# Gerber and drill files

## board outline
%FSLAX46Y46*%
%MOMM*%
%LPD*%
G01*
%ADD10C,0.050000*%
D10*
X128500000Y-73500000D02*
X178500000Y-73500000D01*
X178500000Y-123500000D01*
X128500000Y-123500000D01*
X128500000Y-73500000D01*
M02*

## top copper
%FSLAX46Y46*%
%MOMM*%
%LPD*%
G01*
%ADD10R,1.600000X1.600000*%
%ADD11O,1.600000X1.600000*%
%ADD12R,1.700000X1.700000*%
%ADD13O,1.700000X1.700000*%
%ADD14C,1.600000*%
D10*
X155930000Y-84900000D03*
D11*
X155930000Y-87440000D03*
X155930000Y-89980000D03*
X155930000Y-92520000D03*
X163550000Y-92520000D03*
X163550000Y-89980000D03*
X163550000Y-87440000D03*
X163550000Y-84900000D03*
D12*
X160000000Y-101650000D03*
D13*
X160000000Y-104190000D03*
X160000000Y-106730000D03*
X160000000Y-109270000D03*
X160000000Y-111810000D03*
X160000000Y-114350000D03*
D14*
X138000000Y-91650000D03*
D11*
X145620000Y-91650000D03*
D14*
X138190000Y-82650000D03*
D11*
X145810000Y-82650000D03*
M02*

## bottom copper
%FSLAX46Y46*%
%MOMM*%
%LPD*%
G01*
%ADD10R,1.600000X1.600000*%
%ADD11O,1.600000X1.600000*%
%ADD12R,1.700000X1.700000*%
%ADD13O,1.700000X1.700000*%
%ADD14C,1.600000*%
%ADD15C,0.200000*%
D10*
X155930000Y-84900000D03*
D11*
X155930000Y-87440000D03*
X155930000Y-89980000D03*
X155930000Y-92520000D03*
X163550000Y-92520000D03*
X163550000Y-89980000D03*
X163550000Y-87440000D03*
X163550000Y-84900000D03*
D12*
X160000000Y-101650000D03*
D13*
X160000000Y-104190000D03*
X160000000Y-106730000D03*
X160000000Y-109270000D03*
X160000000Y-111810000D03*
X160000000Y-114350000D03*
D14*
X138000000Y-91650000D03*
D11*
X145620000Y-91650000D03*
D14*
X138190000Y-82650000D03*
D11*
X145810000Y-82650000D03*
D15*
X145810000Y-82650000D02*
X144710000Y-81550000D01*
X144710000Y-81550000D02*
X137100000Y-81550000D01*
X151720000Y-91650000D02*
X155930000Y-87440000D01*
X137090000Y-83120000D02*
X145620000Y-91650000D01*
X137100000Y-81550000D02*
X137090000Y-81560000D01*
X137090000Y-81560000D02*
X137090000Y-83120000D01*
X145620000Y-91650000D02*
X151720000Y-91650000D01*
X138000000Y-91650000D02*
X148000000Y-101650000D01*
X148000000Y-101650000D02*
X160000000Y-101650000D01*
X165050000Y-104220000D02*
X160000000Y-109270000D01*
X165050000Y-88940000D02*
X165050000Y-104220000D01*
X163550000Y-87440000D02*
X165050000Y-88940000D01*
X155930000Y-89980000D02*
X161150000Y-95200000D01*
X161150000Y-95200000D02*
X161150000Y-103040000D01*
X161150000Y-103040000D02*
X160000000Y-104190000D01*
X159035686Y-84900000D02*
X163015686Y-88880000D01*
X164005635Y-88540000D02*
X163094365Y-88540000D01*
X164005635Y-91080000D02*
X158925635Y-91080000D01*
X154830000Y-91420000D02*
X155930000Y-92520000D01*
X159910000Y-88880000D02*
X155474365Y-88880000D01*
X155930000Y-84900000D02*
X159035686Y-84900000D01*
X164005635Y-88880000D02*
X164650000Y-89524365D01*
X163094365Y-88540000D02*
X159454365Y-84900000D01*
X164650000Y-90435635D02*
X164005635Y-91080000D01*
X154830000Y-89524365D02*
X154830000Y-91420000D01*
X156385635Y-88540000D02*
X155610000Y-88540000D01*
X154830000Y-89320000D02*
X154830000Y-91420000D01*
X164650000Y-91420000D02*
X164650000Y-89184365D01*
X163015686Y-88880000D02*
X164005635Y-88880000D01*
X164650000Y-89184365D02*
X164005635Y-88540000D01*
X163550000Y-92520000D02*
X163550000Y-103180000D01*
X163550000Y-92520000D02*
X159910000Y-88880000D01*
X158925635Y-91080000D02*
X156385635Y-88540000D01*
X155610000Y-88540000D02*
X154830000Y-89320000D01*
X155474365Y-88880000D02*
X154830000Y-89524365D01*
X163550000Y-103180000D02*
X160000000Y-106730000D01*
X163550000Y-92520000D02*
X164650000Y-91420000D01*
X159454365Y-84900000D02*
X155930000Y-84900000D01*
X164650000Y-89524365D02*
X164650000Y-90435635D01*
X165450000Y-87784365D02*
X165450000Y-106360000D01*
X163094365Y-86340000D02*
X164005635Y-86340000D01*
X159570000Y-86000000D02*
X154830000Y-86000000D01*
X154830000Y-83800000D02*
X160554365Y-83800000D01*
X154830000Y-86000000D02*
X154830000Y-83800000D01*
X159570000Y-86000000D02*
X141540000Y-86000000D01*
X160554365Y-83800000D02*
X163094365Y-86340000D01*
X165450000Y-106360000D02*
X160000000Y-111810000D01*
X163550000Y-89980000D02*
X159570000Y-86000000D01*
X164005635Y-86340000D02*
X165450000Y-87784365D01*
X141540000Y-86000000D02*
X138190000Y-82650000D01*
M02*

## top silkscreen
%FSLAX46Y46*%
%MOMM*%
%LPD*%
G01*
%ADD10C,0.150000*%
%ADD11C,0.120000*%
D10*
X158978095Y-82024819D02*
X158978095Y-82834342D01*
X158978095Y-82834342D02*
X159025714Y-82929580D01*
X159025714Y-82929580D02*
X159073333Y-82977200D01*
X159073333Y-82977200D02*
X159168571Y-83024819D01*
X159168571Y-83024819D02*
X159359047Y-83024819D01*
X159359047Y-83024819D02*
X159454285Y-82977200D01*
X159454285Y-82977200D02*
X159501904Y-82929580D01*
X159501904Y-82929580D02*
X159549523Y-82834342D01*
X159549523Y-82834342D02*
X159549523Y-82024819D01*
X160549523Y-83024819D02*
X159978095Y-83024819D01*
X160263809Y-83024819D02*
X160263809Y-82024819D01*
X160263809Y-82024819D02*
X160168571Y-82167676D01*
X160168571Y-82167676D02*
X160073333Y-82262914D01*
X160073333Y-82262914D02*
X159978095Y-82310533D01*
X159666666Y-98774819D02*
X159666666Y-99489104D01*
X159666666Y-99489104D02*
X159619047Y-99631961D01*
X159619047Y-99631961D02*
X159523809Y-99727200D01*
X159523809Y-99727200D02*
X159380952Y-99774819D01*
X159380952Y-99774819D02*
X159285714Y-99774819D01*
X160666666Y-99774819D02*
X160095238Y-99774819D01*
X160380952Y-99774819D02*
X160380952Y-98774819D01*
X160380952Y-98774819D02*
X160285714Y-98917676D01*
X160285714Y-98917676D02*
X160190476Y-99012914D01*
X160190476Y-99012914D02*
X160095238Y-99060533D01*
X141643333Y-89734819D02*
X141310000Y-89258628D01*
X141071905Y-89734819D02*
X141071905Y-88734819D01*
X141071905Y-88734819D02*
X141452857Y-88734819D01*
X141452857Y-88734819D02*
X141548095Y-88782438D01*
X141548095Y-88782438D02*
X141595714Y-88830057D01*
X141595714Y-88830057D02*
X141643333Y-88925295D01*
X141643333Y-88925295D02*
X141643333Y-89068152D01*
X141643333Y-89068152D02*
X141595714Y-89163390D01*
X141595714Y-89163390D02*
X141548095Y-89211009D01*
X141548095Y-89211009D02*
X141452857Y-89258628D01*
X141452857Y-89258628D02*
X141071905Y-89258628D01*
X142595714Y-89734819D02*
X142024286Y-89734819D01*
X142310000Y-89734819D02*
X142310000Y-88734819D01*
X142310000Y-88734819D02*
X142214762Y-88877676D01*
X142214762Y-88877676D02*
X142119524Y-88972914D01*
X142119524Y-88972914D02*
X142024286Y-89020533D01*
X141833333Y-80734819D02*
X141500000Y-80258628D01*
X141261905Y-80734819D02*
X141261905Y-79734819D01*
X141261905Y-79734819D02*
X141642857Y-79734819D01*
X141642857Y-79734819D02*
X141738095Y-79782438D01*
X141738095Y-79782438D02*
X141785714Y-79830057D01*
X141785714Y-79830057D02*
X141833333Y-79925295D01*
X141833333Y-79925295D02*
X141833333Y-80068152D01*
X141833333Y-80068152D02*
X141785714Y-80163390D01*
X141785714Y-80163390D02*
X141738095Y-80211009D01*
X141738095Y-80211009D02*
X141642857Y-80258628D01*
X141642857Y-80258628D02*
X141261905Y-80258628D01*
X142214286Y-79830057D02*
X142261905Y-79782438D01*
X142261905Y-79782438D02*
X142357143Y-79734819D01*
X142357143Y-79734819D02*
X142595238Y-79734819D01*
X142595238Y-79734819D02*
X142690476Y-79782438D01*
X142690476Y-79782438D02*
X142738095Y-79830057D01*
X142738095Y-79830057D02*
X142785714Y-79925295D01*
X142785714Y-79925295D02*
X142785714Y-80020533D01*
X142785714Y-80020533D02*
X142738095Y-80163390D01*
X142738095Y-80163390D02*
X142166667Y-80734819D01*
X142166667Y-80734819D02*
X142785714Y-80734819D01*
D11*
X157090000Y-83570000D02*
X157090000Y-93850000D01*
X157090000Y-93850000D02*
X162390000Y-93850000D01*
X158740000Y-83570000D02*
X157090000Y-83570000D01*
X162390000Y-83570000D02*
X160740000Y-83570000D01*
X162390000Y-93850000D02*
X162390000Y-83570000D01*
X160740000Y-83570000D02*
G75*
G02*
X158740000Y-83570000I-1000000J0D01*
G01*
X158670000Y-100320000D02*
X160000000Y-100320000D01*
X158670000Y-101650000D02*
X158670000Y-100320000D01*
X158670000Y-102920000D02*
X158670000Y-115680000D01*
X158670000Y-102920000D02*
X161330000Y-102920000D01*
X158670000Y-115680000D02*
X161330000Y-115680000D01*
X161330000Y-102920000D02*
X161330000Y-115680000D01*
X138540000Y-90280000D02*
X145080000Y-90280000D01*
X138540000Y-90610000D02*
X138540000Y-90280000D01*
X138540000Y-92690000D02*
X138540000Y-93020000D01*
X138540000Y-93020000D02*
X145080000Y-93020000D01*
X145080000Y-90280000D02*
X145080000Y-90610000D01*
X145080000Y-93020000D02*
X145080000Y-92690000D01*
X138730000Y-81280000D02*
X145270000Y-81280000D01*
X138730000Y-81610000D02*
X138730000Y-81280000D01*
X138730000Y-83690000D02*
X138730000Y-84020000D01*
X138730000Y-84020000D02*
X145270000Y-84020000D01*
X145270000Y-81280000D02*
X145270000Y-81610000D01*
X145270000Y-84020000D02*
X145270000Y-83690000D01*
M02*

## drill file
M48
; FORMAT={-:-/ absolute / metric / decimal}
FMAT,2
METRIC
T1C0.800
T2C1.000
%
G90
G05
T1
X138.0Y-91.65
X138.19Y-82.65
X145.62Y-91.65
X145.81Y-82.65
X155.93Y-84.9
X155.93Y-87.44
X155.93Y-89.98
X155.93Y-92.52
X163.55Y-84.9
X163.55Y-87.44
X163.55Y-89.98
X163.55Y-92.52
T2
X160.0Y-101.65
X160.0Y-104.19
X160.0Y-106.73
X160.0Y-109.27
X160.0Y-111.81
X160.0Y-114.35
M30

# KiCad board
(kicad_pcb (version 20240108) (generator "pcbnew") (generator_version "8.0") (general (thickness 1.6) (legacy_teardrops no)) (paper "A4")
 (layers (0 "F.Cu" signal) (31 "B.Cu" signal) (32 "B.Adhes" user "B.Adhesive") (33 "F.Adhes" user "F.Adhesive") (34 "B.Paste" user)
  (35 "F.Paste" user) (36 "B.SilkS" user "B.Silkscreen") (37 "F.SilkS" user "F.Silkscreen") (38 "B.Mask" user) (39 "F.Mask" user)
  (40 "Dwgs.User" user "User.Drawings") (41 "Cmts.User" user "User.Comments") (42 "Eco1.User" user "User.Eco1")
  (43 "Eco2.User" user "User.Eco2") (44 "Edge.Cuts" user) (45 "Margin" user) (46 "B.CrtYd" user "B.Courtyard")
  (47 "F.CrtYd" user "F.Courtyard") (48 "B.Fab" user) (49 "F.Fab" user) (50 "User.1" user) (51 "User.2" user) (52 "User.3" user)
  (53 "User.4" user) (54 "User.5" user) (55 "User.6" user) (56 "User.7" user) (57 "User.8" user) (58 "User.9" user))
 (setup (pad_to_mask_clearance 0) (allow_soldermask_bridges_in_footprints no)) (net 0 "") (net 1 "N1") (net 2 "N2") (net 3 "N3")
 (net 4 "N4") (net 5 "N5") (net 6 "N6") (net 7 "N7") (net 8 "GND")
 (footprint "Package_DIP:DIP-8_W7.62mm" (layer "F.Cu") (at 155.93 84.9)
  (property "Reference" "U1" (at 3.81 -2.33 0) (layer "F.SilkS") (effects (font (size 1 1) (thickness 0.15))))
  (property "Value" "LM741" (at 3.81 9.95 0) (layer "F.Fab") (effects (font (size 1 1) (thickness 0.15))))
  (fp_line (start 1.16 -1.33) (end 1.16 8.95) (stroke (width 0.12) (type solid)) (layer "F.SilkS"))
  (fp_line (start 1.16 8.95) (end 6.46 8.95) (stroke (width 0.12) (type solid)) (layer "F.SilkS"))
  (fp_line (start 2.81 -1.33) (end 1.16 -1.33) (stroke (width 0.12) (type solid)) (layer "F.SilkS"))
  (fp_line (start 6.46 -1.33) (end 4.81 -1.33) (stroke (width 0.12) (type solid)) (layer "F.SilkS"))
  (fp_line (start 6.46 8.95) (end 6.46 -1.33) (stroke (width 0.12) (type solid)) (layer "F.SilkS"))
  (fp_arc (start 4.81 -1.33) (mid 3.81 -0.33) (end 2.81 -1.33) (stroke (width 0.12) (type solid)) (layer "F.SilkS"))
  (pad "1" thru_hole rect (at 0 0) (size 1.6 1.6) (drill 0.8) (layers "*.Cu" "*.Mask") (remove_unused_layers no) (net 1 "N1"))
  (pad "2" thru_hole oval (at 0 2.54) (size 1.6 1.6) (drill 0.8) (layers "*.Cu" "*.Mask") (remove_unused_layers no) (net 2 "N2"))
  (pad "3" thru_hole oval (at 0 5.08) (size 1.6 1.6) (drill 0.8) (layers "*.Cu" "*.Mask") (remove_unused_layers no) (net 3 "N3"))
  (pad "4" thru_hole oval (at 0 7.62) (size 1.6 1.6) (drill 0.8) (layers "*.Cu" "*.Mask") (remove_unused_layers no) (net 1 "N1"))
  (pad "5" thru_hole oval (at 7.62 7.62) (size 1.6 1.6) (drill 0.8) (layers "*.Cu" "*.Mask") (remove_unused_layers no) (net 1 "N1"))
  (pad "6" thru_hole oval (at 7.62 5.08) (size 1.6 1.6) (drill 0.8) (layers "*.Cu" "*.Mask") (remove_unused_layers no) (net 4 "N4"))
  (pad "7" thru_hole oval (at 7.62 2.54) (size 1.6 1.6) (drill 0.8) (layers "*.Cu" "*.Mask") (remove_unused_layers no) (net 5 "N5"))
  (pad "8" thru_hole oval (at 7.62 0) (size 1.6 1.6) (drill 0.8) (layers "*.Cu" "*.Mask") (remove_unused_layers no) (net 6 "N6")))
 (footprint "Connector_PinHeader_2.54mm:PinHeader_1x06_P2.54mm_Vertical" (layer "F.Cu") (at 160 101.65)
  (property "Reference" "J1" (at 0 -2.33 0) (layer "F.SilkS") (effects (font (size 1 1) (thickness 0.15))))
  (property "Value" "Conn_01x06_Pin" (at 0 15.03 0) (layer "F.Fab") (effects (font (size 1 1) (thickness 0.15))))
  (fp_line (start -1.33 -1.33) (end 0 -1.33) (stroke (width 0.12) (type solid)) (layer "F.SilkS"))
  (fp_line (start -1.33 0) (end -1.33 -1.33) (stroke (width 0.12) (type solid)) (layer "F.SilkS"))
  (fp_line (start -1.33 1.27) (end -1.33 14.03) (stroke (width 0.12) (type solid)) (layer "F.SilkS"))
  (fp_line (start -1.33 1.27) (end 1.33 1.27) (stroke (width 0.12) (type solid)) (layer "F.SilkS"))
  (fp_line (start -1.33 14.03) (end 1.33 14.03) (stroke (width 0.12) (type solid)) (layer "F.SilkS"))
  (fp_line (start 1.33 1.27) (end 1.33 14.03) (stroke (width 0.12) (type solid)) (layer "F.SilkS"))
  (pad "1" thru_hole rect (at 0 0) (size 1.7 1.7) (drill 1) (layers "*.Cu" "*.Mask") (remove_unused_layers no) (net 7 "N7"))
  (pad "2" thru_hole oval (at 0 2.54) (size 1.7 1.7) (drill 1) (layers "*.Cu" "*.Mask") (remove_unused_layers no) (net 3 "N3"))
  (pad "3" thru_hole oval (at 0 5.08) (size 1.7 1.7) (drill 1) (layers "*.Cu" "*.Mask") (remove_unused_layers no) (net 1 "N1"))
  (pad "4" thru_hole oval (at 0 7.62) (size 1.7 1.7) (drill 1) (layers "*.Cu" "*.Mask") (remove_unused_layers no) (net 5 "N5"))
  (pad "5" thru_hole oval (at 0 10.16) (size 1.7 1.7) (drill 1) (layers "*.Cu" "*.Mask") (remove_unused_layers no) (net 4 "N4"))
  (pad "6" thru_hole oval (at 0 12.7) (size 1.7 1.7) (drill 1) (layers "*.Cu" "*.Mask") (remove_unused_layers no) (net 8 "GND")))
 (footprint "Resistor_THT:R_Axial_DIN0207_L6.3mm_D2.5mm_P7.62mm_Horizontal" (layer "F.Cu") (at 138 91.65)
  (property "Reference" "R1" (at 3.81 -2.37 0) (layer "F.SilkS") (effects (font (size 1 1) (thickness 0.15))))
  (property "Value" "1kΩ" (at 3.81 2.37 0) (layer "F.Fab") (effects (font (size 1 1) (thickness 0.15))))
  (fp_line (start 0.54 -1.37) (end 7.08 -1.37) (stroke (width 0.12) (type solid)) (layer "F.SilkS"))
  (fp_line (start 0.54 -1.04) (end 0.54 -1.37) (stroke (width 0.12) (type solid)) (layer "F.SilkS"))
  (fp_line (start 0.54 1.04) (end 0.54 1.37) (stroke (width 0.12) (type solid)) (layer "F.SilkS"))
  (fp_line (start 0.54 1.37) (end 7.08 1.37) (stroke (width 0.12) (type solid)) (layer "F.SilkS"))
  (fp_line (start 7.08 -1.37) (end 7.08 -1.04) (stroke (width 0.12) (type solid)) (layer "F.SilkS"))
  (fp_line (start 7.08 1.37) (end 7.08 1.04) (stroke (width 0.12) (type solid)) (layer "F.SilkS"))
  (pad "1" thru_hole circle (at 0 0) (size 1.6 1.6) (drill 0.8) (layers "*.Cu" "*.Mask") (remove_unused_layers no) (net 7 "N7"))
  (pad "2" thru_hole oval (at 7.62 0) (size 1.6 1.6) (drill 0.8) (layers "*.Cu" "*.Mask") (remove_unused_layers no) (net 2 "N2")))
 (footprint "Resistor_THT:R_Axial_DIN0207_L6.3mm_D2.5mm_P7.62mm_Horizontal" (layer "F.Cu") (at 138.19 82.65)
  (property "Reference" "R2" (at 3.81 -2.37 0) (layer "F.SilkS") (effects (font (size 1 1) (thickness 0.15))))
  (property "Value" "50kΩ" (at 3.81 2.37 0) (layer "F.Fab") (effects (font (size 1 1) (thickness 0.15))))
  (fp_line (start 0.54 -1.37) (end 7.08 -1.37) (stroke (width 0.12) (type solid)) (layer "F.SilkS"))
  (fp_line (start 0.54 -1.04) (end 0.54 -1.37) (stroke (width 0.12) (type solid)) (layer "F.SilkS"))
  (fp_line (start 0.54 1.04) (end 0.54 1.37) (stroke (width 0.12) (type solid)) (layer "F.SilkS"))
  (fp_line (start 0.54 1.37) (end 7.08 1.37) (stroke (width 0.12) (type solid)) (layer "F.SilkS"))
  (fp_line (start 7.08 -1.37) (end 7.08 -1.04) (stroke (width 0.12) (type solid)) (layer "F.SilkS"))
  (fp_line (start 7.08 1.37) (end 7.08 1.04) (stroke (width 0.12) (type solid)) (layer "F.SilkS"))
  (pad "1" thru_hole circle (at 0 0) (size 1.6 1.6) (drill 0.8) (layers "*.Cu" "*.Mask") (remove_unused_layers no) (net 4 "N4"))
  (pad "2" thru_hole oval (at 7.62 0) (size 1.6 1.6) (drill 0.8) (layers "*.Cu" "*.Mask") (remove_unused_layers no) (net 2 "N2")))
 (gr_rect (start 128.5 73.5) (end 178.5 123.5) (stroke (width 0.05) (type default)) (fill none) (layer "Edge.Cuts"))
 (segment (start 145.81 82.65) (end 144.71 81.55) (width 0.2) (layer "B.Cu") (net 2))
 (segment (start 144.71 81.55) (end 137.1 81.55) (width 0.2) (layer "B.Cu") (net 2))
 (segment (start 151.72 91.65) (end 155.93 87.44) (width 0.2) (layer "B.Cu") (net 2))
 (segment (start 137.09 83.12) (end 145.62 91.65) (width 0.2) (layer "B.Cu") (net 2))
 (segment (start 137.1 81.55) (end 137.09 81.56) (width 0.2) (layer "B.Cu") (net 2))
 (segment (start 137.09 81.56) (end 137.09 83.12) (width 0.2) (layer "B.Cu") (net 2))
 (segment (start 145.62 91.65) (end 151.72 91.65) (width 0.2) (layer "B.Cu") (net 2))
 (segment (start 138 91.65) (end 148 101.65) (width 0.2) (layer "B.Cu") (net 7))
 (segment (start 148 101.65) (end 160 101.65) (width 0.2) (layer "B.Cu") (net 7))
 (segment (start 165.05 104.22) (end 160 109.27) (width 0.2) (layer "B.Cu") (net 5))
 (segment (start 165.05 88.94) (end 165.05 104.22) (width 0.2) (layer "B.Cu") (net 5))
 (segment (start 163.55 87.44) (end 165.05 88.94) (width 0.2) (layer "B.Cu") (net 5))
 (segment (start 155.93 89.98) (end 161.15 95.2) (width 0.2) (layer "B.Cu") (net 3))
 (segment (start 161.15 95.2) (end 161.15 103.04) (width 0.2) (layer "B.Cu") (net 3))
 (segment (start 161.15 103.04) (end 160 104.19) (width 0.2) (layer "B.Cu") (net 3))
 (segment (start 159.035686 84.9) (end 163.015686 88.88) (width 0.2) (layer "B.Cu") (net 1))
 (segment (start 164.005635 88.54) (end 163.094365 88.54) (width 0.2) (layer "B.Cu") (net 1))
 (segment (start 164.005635 91.08) (end 158.925635 91.08) (width 0.2) (layer "B.Cu") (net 1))
 (segment (start 154.83 91.42) (end 155.93 92.52) (width 0.2) (layer "B.Cu") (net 1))
 (segment (start 159.91 88.88) (end 155.474365 88.88) (width 0.2) (layer "B.Cu") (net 1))
 (segment (start 155.93 84.9) (end 159.035686 84.9) (width 0.2) (layer "B.Cu") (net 1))
 (segment (start 164.005635 88.88) (end 164.65 89.524365) (width 0.2) (layer "B.Cu") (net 1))
 (segment (start 163.094365 88.54) (end 159.454365 84.9) (width 0.2) (layer "B.Cu") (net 1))
 (segment (start 164.65 90.435635) (end 164.005635 91.08) (width 0.2) (layer "B.Cu") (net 1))
 (segment (start 154.83 89.524365) (end 154.83 91.42) (width 0.2) (layer "B.Cu") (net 1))
 (segment (start 156.385635 88.54) (end 155.61 88.54) (width 0.2) (layer "B.Cu") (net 1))
 (segment (start 154.83 89.32) (end 154.83 91.42) (width 0.2) (layer "B.Cu") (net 1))
 (segment (start 164.65 91.42) (end 164.65 89.184365) (width 0.2) (layer "B.Cu") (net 1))
 (segment (start 163.015686 88.88) (end 164.005635 88.88) (width 0.2) (layer "B.Cu") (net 1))
 (segment (start 164.65 89.184365) (end 164.005635 88.54) (width 0.2) (layer "B.Cu") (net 1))
 (segment (start 163.55 92.52) (end 163.55 103.18) (width 0.2) (layer "B.Cu") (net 1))
 (segment (start 163.55 92.52) (end 159.91 88.88) (width 0.2) (layer "B.Cu") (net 1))
 (segment (start 158.925635 91.08) (end 156.385635 88.54) (width 0.2) (layer "B.Cu") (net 1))
 (segment (start 155.61 88.54) (end 154.83 89.32) (width 0.2) (layer "B.Cu") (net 1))
 (segment (start 155.474365 88.88) (end 154.83 89.524365) (width 0.2) (layer "B.Cu") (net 1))
 (segment (start 163.55 103.18) (end 160 106.73) (width 0.2) (layer "B.Cu") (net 1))
 (segment (start 163.55 92.52) (end 164.65 91.42) (width 0.2) (layer "B.Cu") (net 1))
 (segment (start 159.454365 84.9) (end 155.93 84.9) (width 0.2) (layer "B.Cu") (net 1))
 (segment (start 164.65 89.524365) (end 164.65 90.435635) (width 0.2) (layer "B.Cu") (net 1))
 (segment (start 165.45 87.784365) (end 165.45 106.36) (width 0.2) (layer "B.Cu") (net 4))
 (segment (start 163.094365 86.34) (end 164.005635 86.34) (width 0.2) (layer "B.Cu") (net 4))
 (segment (start 159.57 86) (end 154.83 86) (width 0.2) (layer "B.Cu") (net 4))
 (segment (start 154.83 83.8) (end 160.554365 83.8) (width 0.2) (layer "B.Cu") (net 4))
 (segment (start 154.83 86) (end 154.83 83.8) (width 0.2) (layer "B.Cu") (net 4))
 (segment (start 159.57 86) (end 141.54 86) (width 0.2) (layer "B.Cu") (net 4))
 (segment (start 160.554365 83.8) (end 163.094365 86.34) (width 0.2) (layer "B.Cu") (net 4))
 (segment (start 165.45 106.36) (end 160 111.81) (width 0.2) (layer "B.Cu") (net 4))
 (segment (start 163.55 89.98) (end 159.57 86) (width 0.2) (layer "B.Cu") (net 4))
 (segment (start 164.005635 86.34) (end 165.45 87.784365) (width 0.2) (layer "B.Cu") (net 4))
 (segment (start 141.54 86) (end 138.19 82.65) (width 0.2) (layer "B.Cu") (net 4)))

